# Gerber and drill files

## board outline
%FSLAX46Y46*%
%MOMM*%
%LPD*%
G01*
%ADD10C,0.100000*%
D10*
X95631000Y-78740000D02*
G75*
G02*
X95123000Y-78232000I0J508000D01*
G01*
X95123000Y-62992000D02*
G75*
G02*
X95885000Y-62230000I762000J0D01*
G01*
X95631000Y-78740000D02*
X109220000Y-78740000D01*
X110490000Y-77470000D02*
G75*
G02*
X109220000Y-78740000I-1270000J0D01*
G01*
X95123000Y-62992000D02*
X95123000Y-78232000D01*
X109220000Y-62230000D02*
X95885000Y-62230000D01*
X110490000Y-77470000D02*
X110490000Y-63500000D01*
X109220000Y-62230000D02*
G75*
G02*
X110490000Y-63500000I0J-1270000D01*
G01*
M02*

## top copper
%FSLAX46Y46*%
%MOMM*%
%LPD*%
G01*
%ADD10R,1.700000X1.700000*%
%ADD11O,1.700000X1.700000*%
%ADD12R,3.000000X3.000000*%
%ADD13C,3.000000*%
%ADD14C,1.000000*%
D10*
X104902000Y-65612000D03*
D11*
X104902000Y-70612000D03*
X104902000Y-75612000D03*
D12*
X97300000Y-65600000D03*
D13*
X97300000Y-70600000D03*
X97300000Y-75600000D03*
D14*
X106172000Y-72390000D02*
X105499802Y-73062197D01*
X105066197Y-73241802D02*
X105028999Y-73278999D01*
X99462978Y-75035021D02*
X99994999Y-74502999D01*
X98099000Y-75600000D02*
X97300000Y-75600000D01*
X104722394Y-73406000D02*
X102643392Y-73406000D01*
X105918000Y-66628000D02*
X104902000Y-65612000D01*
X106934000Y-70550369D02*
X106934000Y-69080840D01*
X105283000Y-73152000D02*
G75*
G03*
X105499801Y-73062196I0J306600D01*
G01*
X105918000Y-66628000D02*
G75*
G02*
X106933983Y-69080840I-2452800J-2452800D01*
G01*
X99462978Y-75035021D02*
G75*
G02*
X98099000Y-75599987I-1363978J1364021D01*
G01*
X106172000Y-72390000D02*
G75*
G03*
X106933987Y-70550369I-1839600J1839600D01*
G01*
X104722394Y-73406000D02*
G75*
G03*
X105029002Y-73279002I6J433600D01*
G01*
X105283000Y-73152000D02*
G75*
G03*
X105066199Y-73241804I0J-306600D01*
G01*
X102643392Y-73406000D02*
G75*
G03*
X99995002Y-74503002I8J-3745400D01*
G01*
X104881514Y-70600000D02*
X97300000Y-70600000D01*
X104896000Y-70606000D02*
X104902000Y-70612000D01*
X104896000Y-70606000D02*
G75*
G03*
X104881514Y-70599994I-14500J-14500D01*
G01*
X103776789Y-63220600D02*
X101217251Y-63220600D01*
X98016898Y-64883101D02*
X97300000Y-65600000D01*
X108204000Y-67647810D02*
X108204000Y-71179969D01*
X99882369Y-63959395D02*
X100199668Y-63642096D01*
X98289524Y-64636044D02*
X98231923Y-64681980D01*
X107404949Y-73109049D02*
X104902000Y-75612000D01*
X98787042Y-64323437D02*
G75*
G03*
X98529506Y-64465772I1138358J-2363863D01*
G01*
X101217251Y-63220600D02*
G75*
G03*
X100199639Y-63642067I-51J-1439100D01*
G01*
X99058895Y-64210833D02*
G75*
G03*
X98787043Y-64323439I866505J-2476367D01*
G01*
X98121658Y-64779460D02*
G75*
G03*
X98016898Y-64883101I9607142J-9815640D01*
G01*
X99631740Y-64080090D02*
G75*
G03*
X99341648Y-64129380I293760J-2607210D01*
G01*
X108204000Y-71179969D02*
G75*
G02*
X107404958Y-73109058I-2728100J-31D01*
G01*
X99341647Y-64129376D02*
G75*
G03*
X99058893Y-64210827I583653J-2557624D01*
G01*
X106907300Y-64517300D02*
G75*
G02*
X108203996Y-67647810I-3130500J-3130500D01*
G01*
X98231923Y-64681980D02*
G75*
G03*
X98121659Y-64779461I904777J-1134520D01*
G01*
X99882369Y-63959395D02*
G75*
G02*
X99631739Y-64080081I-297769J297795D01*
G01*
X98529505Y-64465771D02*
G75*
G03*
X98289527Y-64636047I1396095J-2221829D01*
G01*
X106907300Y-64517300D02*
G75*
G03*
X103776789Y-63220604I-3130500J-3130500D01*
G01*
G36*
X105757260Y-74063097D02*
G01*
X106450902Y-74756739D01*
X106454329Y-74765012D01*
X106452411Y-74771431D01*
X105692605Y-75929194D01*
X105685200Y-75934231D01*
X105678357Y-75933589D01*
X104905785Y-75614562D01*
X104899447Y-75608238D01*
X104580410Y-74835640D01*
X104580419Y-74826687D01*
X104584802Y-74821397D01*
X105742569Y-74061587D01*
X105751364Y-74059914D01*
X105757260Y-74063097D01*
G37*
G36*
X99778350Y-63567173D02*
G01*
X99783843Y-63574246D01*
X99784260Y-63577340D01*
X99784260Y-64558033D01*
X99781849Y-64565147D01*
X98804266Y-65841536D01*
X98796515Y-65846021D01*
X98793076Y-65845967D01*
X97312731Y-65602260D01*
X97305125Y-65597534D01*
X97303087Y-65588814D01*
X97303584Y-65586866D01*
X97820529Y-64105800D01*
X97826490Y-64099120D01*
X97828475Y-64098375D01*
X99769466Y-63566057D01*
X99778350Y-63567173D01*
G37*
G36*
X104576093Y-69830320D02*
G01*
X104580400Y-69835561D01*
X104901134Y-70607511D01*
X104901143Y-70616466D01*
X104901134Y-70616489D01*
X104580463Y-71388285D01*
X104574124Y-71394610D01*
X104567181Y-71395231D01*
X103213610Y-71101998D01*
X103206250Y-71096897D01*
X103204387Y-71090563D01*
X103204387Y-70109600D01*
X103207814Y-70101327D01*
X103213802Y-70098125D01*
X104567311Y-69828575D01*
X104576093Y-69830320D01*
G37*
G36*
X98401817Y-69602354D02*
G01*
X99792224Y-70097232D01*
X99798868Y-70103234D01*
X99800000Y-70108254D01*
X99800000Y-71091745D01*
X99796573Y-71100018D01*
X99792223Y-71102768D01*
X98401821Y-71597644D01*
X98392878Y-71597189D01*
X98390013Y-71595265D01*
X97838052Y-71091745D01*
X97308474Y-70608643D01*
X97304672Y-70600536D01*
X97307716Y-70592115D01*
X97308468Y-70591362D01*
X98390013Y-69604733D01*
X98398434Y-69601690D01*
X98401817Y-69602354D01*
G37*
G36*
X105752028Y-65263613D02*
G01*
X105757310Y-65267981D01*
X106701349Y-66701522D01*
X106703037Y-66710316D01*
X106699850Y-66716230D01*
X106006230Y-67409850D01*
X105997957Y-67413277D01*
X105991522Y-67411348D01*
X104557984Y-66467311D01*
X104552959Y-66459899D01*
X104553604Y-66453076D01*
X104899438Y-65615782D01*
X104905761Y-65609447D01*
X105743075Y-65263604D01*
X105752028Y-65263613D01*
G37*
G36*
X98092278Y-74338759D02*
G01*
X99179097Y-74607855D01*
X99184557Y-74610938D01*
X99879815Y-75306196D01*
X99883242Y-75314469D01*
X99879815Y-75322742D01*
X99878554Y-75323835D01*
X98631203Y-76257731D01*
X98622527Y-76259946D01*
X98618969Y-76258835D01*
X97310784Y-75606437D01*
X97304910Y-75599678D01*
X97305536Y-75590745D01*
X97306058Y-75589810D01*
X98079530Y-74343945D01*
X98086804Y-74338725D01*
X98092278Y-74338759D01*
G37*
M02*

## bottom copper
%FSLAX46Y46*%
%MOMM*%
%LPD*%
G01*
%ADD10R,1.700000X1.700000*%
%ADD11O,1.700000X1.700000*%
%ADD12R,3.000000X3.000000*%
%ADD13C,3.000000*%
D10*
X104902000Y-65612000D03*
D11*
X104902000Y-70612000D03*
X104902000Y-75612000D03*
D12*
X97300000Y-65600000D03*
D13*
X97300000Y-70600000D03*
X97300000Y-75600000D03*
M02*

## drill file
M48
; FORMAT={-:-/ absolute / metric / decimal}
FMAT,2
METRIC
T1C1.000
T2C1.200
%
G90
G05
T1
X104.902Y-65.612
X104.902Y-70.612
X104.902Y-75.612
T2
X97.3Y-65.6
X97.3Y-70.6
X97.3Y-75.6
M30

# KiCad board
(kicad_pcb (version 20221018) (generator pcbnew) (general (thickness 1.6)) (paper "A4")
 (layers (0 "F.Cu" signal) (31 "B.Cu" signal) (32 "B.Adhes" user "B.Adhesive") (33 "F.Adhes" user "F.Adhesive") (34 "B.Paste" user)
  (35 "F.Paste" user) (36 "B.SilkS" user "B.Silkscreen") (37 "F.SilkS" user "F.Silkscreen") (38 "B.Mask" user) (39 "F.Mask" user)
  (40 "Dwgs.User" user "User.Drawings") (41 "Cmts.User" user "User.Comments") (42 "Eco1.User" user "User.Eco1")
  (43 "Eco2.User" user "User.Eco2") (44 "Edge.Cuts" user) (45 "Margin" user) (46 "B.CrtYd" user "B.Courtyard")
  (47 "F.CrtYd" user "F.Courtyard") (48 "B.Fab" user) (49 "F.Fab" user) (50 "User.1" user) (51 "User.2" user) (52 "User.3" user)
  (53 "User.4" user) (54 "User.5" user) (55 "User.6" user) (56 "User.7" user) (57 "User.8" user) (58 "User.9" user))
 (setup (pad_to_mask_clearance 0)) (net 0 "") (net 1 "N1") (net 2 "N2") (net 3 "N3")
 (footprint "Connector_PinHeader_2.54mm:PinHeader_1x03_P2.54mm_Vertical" (layer "F.Cu") (at 104.902 70.612)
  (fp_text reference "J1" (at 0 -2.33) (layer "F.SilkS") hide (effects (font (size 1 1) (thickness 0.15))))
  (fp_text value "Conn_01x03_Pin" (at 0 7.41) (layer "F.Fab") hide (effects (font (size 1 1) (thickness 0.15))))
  (pad "1" thru_hole rect (at 0 -5) (size 1.7 1.7) (drill 1) (layers "*.Cu" "*.Mask") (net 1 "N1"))
  (pad "2" thru_hole oval (at 0 0) (size 1.7 1.7) (drill 1) (layers "*.Cu" "*.Mask") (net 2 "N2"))
  (pad "3" thru_hole oval (at 0 5) (size 1.7 1.7) (drill 1) (layers "*.Cu" "*.Mask") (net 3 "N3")))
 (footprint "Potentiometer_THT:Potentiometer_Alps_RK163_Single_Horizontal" (layer "F.Cu") (at 97.3 65.6)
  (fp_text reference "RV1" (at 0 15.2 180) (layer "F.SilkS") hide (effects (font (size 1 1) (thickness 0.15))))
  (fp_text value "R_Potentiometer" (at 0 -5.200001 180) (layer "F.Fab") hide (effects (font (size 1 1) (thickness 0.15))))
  (pad "1" thru_hole rect (at 0 0 180) (size 3 3) (drill 1.2) (layers "*.Cu" "*.Mask") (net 3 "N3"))
  (pad "2" thru_hole circle (at 0 5 180) (size 3 3) (drill 1.2) (layers "*.Cu" "*.Mask") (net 2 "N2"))
  (pad "3" thru_hole circle (at 0 10 180) (size 3 3) (drill 1.2) (layers "*.Cu" "*.Mask") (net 1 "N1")))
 (gr_arc (start 95.631 78.74) (mid 95.27179 78.59121) (end 95.123 78.232) (stroke (width 0.1) (type default)) (layer "Edge.Cuts"))
 (gr_arc (start 95.123 62.992) (mid 95.346185 62.453185) (end 95.885 62.23) (stroke (width 0.1) (type default)) (layer "Edge.Cuts"))
 (gr_line (start 95.631 78.74) (end 109.22 78.74) (stroke (width 0.1) (type default)) (layer "Edge.Cuts"))
 (gr_arc (start 110.49 77.47) (mid 110.118026 78.368026) (end 109.22 78.74) (stroke (width 0.1) (type default)) (layer "Edge.Cuts"))
 (gr_line (start 95.123 62.992) (end 95.123 78.232) (stroke (width 0.1) (type default)) (layer "Edge.Cuts"))
 (gr_line (start 109.22 62.23) (end 95.885 62.23) (stroke (width 0.1) (type default)) (layer "Edge.Cuts"))
 (gr_line (start 110.49 77.47) (end 110.49 63.5) (stroke (width 0.1) (type default)) (layer "Edge.Cuts"))
 (gr_arc (start 109.22 62.23) (mid 110.118026 62.601974) (end 110.49 63.5) (stroke (width 0.1) (type default)) (layer "Edge.Cuts"))
 (segment (start 106.172 72.39) (end 105.499802 73.062197) (width 1) (layer "F.Cu") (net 1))
 (segment (start 105.066197 73.241802) (end 105.028999 73.278999) (width 1) (layer "F.Cu") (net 1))
 (segment (start 99.462978 75.035021) (end 99.994999 74.502999) (width 1) (layer "F.Cu") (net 1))
 (segment (start 98.099 75.6) (end 97.3 75.6) (width 1) (layer "F.Cu") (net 1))
 (segment (start 104.722394 73.406) (end 102.643392 73.406) (width 1) (layer "F.Cu") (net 1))
 (segment (start 105.918 66.628) (end 104.902 65.612) (width 1) (layer "F.Cu") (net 1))
 (segment (start 106.934 70.550369) (end 106.934 69.08084) (width 1) (layer "F.Cu") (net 1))
 (arc (start 105.283 73.152) (mid 105.400332 73.12866) (end 105.499802 73.062197) (width 1) (layer "F.Cu") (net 1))
 (arc (start 105.918 66.628) (mid 106.66995 67.753372) (end 106.934 69.08084) (width 1) (layer "F.Cu") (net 1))
 (arc (start 99.462978 75.035021) (mid 98.837179 75.453166) (end 98.099 75.6) (width 1) (layer "F.Cu") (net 1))
 (arc (start 106.172 72.39) (mid 106.735962 71.54597) (end 106.934 70.550369) (width 1) (layer "F.Cu") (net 1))
 (arc (start 104.722394 73.406) (mid 104.888327 73.372993) (end 105.028999 73.278999) (width 1) (layer "F.Cu") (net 1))
 (arc (start 105.283 73.152) (mid 105.165667 73.175338) (end 105.066197 73.241802) (width 1) (layer "F.Cu") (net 1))
 (arc (start 102.643392 73.406) (mid 101.210092 73.6911) (end 99.994999 74.502999) (width 1) (layer "F.Cu") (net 1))
 (segment (start 104.881514 70.6) (end 97.3 70.6) (width 1) (layer "F.Cu") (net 2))
 (segment (start 104.896 70.606) (end 104.902 70.612) (width 1) (layer "F.Cu") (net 2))
 (arc (start 104.896 70.606) (mid 104.889353 70.601559) (end 104.881514 70.6) (width 1) (layer "F.Cu") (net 2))
 (segment (start 103.776789 63.2206) (end 101.217251 63.2206) (width 1) (layer "F.Cu") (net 3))
 (segment (start 98.016898 64.883101) (end 97.3 65.6) (width 1) (layer "F.Cu") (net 3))
 (segment (start 108.204 67.64781) (end 108.204 71.179969) (width 1) (layer "F.Cu") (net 3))
 (segment (start 99.882369 63.959395) (end 100.199668 63.642096) (width 1) (layer "F.Cu") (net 3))
 (segment (start 98.289524 64.636044) (end 98.231923 64.68198) (width 1) (layer "F.Cu") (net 3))
 (segment (start 107.404949 73.109049) (end 104.902 75.612) (width 1) (layer "F.Cu") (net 3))
 (arc (start 98.787042 64.323437) (mid 98.656276 64.390991) (end 98.529505 64.465771) (width 1) (layer "F.Cu") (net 3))
 (arc (start 101.217251 63.2206) (mid 100.666539 63.330143) (end 100.199668 63.642096) (width 1) (layer "F.Cu") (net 3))
 (arc (start 99.058895 64.210833) (mid 98.921388 64.263321) (end 98.787042 64.323437) (width 1) (layer "F.Cu") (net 3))
 (arc (start 98.121658 64.77946) (mid 98.069139 64.83114) (end 98.016898 64.883101) (width 1) (layer "F.Cu") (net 3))
 (arc (start 99.63174 64.08009) (mid 99.486002 64.100663) (end 99.341647 64.129376) (width 1) (layer "F.Cu") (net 3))
 (arc (start 108.204 71.179969) (mid 107.996333 72.22398) (end 107.404949 73.109049) (width 1) (layer "F.Cu") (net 3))
 (arc (start 99.341647 64.129376) (mid 99.199128 64.166137) (end 99.058895 64.210833) (width 1) (layer "F.Cu") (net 3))
 (arc (start 106.9073 64.5173) (mid 107.866998 65.95359) (end 108.204 67.64781) (width 1) (layer "F.Cu") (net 3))
 (arc (start 98.231923 64.68198) (mid 98.175554 64.729321) (end 98.121658 64.77946) (width 1) (layer "F.Cu") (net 3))
 (arc (start 99.882369 63.959395) (mid 99.767308 64.041034) (end 99.63174 64.08009) (width 1) (layer "F.Cu") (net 3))
 (arc (start 98.529505 64.465771) (mid 98.407126 64.547541) (end 98.289524 64.636044) (width 1) (layer "F.Cu") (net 3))
 (arc (start 106.9073 64.5173) (mid 105.471009 63.557601) (end 103.776789 63.2206) (width 1) (layer "F.Cu") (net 3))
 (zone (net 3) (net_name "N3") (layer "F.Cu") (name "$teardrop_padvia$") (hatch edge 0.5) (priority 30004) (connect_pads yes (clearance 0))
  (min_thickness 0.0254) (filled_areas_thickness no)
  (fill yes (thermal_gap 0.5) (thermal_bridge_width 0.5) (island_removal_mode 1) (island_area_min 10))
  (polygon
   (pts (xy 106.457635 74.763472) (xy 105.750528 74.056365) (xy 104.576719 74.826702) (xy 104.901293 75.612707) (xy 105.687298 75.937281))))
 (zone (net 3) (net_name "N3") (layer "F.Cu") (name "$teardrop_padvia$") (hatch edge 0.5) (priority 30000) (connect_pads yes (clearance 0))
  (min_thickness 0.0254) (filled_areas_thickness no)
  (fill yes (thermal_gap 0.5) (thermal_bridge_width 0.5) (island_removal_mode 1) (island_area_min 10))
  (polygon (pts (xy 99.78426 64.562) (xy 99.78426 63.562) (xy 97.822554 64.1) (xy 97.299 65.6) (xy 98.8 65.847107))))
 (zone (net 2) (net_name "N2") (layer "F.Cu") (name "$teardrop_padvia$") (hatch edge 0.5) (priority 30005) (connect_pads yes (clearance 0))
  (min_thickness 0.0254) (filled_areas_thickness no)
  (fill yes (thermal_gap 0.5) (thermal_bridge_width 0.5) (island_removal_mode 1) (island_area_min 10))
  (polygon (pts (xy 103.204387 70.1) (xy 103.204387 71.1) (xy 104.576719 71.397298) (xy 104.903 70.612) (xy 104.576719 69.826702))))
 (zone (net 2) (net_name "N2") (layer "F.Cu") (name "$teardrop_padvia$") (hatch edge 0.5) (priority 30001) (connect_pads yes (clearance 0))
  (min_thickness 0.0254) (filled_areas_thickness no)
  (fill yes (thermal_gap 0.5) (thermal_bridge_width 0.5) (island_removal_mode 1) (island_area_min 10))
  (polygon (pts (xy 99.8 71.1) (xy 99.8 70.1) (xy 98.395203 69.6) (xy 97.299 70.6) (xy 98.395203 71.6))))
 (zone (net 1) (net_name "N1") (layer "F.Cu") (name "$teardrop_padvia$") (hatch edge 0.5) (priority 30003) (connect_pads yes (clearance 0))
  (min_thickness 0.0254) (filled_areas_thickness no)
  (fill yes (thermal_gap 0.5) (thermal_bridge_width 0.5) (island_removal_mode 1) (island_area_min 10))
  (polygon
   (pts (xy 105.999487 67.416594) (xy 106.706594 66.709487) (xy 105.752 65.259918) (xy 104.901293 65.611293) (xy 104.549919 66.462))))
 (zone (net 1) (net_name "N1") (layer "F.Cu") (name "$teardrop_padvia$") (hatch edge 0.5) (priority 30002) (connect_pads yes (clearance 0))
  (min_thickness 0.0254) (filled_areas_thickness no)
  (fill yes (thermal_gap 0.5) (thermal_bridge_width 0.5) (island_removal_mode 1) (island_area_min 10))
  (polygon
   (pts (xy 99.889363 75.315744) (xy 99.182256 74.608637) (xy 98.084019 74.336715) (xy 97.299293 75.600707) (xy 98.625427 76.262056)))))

